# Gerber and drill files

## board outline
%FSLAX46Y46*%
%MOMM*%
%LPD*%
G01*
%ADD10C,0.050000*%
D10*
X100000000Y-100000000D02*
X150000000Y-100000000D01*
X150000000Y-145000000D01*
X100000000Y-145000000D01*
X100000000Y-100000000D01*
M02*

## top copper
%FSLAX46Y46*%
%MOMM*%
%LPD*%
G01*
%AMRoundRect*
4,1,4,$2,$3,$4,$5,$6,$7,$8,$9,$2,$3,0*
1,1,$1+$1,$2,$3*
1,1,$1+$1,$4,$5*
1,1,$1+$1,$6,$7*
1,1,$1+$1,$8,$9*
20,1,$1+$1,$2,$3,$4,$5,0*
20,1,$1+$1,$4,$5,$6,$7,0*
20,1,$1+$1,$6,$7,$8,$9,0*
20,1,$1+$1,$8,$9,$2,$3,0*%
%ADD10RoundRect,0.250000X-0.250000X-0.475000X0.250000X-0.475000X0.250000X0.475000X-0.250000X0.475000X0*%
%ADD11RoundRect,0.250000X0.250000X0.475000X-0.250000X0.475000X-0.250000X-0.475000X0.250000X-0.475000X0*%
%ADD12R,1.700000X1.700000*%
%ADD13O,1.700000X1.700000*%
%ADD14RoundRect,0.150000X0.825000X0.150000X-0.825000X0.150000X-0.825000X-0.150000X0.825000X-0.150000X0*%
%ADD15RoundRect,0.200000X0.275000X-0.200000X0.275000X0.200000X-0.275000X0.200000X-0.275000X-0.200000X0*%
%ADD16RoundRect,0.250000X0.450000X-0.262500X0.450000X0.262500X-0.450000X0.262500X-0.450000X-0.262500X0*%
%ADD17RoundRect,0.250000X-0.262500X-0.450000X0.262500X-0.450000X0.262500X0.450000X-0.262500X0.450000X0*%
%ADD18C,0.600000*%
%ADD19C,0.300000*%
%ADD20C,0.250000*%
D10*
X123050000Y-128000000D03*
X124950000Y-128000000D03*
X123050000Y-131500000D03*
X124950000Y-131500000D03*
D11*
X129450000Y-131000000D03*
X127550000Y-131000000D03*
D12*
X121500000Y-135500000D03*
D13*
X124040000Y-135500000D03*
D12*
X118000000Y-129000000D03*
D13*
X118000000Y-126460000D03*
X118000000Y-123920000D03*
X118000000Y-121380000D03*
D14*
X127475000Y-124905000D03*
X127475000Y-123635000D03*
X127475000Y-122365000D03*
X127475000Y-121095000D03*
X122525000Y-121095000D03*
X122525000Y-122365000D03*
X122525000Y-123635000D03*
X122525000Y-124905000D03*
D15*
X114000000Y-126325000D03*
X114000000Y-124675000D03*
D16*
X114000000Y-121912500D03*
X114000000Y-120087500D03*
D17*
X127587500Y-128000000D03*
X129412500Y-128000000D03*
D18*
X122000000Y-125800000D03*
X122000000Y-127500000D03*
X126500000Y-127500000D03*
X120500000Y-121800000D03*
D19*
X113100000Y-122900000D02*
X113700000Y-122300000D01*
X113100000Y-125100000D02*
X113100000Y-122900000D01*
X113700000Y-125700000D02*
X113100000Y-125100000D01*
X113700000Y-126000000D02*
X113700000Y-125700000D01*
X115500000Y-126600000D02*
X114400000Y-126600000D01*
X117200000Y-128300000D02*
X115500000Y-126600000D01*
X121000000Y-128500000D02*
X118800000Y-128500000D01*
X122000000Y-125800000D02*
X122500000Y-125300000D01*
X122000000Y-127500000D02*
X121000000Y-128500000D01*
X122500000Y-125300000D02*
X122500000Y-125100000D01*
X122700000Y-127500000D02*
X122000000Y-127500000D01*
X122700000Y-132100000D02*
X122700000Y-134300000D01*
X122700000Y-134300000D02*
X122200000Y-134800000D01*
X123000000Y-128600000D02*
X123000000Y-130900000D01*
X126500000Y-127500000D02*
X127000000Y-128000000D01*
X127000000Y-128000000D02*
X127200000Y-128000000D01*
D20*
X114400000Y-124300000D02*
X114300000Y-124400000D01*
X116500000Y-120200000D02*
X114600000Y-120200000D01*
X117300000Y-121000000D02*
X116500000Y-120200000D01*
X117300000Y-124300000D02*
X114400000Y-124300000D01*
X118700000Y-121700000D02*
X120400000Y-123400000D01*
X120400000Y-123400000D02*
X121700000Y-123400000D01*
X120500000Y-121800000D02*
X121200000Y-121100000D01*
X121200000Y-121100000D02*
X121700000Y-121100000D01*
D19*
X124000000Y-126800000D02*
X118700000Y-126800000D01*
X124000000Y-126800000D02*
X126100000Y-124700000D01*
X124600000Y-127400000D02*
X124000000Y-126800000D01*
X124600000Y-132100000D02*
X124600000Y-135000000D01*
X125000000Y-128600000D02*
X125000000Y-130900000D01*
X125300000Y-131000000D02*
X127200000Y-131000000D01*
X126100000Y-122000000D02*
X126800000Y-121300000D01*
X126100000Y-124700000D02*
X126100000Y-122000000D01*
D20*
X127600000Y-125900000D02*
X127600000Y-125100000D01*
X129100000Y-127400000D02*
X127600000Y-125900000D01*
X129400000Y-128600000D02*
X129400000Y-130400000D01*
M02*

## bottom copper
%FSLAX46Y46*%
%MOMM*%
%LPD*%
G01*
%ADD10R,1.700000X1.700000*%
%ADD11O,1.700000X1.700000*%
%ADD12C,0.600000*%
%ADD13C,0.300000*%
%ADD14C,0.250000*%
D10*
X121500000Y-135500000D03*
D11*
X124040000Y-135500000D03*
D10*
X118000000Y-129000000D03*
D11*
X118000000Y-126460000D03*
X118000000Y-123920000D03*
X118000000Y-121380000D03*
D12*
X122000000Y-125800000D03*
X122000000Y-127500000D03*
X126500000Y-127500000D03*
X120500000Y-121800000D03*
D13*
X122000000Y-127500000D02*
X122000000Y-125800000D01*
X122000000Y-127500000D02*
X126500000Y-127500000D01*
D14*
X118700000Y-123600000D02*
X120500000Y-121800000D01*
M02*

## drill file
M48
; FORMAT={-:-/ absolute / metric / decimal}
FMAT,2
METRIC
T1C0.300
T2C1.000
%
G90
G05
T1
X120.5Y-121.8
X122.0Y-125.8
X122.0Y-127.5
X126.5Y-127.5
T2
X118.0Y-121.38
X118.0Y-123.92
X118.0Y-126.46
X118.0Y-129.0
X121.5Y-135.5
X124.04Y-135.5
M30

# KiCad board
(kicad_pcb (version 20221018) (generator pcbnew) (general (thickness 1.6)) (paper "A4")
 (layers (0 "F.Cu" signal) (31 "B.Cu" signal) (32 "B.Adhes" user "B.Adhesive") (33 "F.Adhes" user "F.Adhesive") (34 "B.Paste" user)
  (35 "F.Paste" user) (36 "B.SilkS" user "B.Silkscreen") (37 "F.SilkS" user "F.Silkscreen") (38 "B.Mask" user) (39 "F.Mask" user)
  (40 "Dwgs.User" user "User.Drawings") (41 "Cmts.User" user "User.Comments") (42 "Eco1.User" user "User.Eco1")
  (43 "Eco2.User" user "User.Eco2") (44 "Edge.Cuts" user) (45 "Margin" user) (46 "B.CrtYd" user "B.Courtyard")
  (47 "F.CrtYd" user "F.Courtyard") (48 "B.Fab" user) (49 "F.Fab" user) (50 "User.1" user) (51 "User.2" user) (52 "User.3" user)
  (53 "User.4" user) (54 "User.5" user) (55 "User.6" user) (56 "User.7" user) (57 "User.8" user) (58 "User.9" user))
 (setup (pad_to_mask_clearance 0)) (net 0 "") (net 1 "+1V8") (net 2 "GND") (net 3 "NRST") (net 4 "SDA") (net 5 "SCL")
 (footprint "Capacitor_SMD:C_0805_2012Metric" (layer "F.Cu") (at 124 128)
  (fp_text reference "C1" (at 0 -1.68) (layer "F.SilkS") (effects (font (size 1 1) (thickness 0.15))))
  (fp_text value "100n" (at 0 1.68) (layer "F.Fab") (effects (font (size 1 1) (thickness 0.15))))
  (pad "1" smd roundrect (at -0.95 0) (size 1 1.45) (layers "F.Cu" "F.Paste" "F.Mask") (roundrect_rratio 0.25) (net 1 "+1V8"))
  (pad "2" smd roundrect (at 0.95 0) (size 1 1.45) (layers "F.Cu" "F.Paste" "F.Mask") (roundrect_rratio 0.25) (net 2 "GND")))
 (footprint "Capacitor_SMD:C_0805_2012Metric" (layer "F.Cu") (at 124 131.5)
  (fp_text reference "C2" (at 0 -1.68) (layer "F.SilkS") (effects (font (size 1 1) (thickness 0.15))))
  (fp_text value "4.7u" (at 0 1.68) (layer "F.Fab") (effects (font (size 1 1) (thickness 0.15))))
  (pad "1" smd roundrect (at -0.95 0) (size 1 1.45) (layers "F.Cu" "F.Paste" "F.Mask") (roundrect_rratio 0.25) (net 1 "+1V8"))
  (pad "2" smd roundrect (at 0.95 0) (size 1 1.45) (layers "F.Cu" "F.Paste" "F.Mask") (roundrect_rratio 0.25) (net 2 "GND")))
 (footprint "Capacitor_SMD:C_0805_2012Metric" (layer "F.Cu") (at 128.5 131 180)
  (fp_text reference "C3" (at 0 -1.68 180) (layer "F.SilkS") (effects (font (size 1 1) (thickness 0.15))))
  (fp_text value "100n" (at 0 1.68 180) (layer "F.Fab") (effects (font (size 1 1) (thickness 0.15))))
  (pad "1" smd roundrect (at -0.95 0 180) (size 1 1.45) (layers "F.Cu" "F.Paste" "F.Mask") (roundrect_rratio 0.25) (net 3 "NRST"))
  (pad "2" smd roundrect (at 0.95 0 180) (size 1 1.45) (layers "F.Cu" "F.Paste" "F.Mask") (roundrect_rratio 0.25) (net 2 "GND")))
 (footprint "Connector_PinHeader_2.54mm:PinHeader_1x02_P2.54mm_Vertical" (layer "F.Cu") (at 121.5 135.5 90)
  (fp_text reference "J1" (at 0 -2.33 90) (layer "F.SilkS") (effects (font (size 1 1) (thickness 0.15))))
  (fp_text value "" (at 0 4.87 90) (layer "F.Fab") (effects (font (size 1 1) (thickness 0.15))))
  (pad "1" thru_hole rect (at 0 0 90) (size 1.7 1.7) (drill 1) (layers "*.Cu" "*.Mask") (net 1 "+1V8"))
  (pad "2" thru_hole oval (at 0 2.54 90) (size 1.7 1.7) (drill 1) (layers "*.Cu" "*.Mask") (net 2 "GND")))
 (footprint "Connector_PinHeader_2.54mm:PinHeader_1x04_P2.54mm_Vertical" (layer "F.Cu") (at 118 129 180)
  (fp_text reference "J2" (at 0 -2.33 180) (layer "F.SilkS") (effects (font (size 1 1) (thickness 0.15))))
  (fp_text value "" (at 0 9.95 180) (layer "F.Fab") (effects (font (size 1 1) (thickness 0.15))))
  (pad "1" thru_hole rect (at 0 0 180) (size 1.7 1.7) (drill 1) (layers "*.Cu" "*.Mask") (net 1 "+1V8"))
  (pad "2" thru_hole oval (at 0 2.54 180) (size 1.7 1.7) (drill 1) (layers "*.Cu" "*.Mask") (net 2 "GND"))
  (pad "3" thru_hole oval (at 0 5.08 180) (size 1.7 1.7) (drill 1) (layers "*.Cu" "*.Mask") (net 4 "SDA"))
  (pad "4" thru_hole oval (at 0 7.62 180) (size 1.7 1.7) (drill 1) (layers "*.Cu" "*.Mask") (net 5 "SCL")))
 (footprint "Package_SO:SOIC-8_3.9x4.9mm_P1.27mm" (layer "F.Cu") (at 125 123 180)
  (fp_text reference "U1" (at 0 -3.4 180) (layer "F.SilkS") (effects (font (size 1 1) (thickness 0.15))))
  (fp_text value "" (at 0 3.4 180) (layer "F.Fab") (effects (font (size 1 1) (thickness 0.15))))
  (pad "1" smd roundrect (at -2.475 -1.905 180) (size 1.95 0.6) (layers "F.Cu" "F.Paste" "F.Mask") (roundrect_rratio 0.25) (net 3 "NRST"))
  (pad "2" smd roundrect (at -2.475 -0.635 180) (size 1.95 0.6) (layers "F.Cu" "F.Paste" "F.Mask") (roundrect_rratio 0.25))
  (pad "3" smd roundrect (at -2.475 0.635 180) (size 1.95 0.6) (layers "F.Cu" "F.Paste" "F.Mask") (roundrect_rratio 0.25))
  (pad "4" smd roundrect (at -2.475 1.905 180) (size 1.95 0.6) (layers "F.Cu" "F.Paste" "F.Mask") (roundrect_rratio 0.25) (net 2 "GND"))
  (pad "5" smd roundrect (at 2.475 1.905 180) (size 1.95 0.6) (layers "F.Cu" "F.Paste" "F.Mask") (roundrect_rratio 0.25) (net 4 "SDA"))
  (pad "6" smd roundrect (at 2.475 0.635 180) (size 1.95 0.6) (layers "F.Cu" "F.Paste" "F.Mask") (roundrect_rratio 0.25))
  (pad "7" smd roundrect (at 2.475 -0.635 180) (size 1.95 0.6) (layers "F.Cu" "F.Paste" "F.Mask") (roundrect_rratio 0.25) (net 5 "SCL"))
  (pad "8" smd roundrect (at 2.475 -1.905 180) (size 1.95 0.6) (layers "F.Cu" "F.Paste" "F.Mask") (roundrect_rratio 0.25) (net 1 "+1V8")))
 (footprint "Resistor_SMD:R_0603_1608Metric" (layer "F.Cu") (at 114 125.5 90)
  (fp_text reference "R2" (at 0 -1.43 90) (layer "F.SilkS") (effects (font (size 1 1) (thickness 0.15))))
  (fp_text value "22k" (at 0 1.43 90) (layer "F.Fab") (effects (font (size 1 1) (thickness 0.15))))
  (pad "1" smd roundrect (at -0.825 0 90) (size 0.8 0.95) (layers "F.Cu" "F.Paste" "F.Mask") (roundrect_rratio 0.25) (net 1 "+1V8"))
  (pad "2" smd roundrect (at 0.825 0 90) (size 0.8 0.95) (layers "F.Cu" "F.Paste" "F.Mask") (roundrect_rratio 0.25) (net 4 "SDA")))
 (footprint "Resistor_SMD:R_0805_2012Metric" (layer "F.Cu") (at 114 121 90)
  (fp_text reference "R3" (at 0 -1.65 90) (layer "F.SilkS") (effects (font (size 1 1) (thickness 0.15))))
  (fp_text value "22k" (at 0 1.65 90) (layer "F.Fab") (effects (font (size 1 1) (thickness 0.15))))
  (pad "1" smd roundrect (at -0.9125 0 90) (size 1.025 1.4) (layers "F.Cu" "F.Paste" "F.Mask") (roundrect_rratio 0.243902) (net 1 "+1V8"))
  (pad "2" smd roundrect (at 0.9125 0 90) (size 1.025 1.4) (layers "F.Cu" "F.Paste" "F.Mask") (roundrect_rratio 0.243902) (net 5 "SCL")))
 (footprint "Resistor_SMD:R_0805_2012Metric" (layer "F.Cu") (at 128.5 128)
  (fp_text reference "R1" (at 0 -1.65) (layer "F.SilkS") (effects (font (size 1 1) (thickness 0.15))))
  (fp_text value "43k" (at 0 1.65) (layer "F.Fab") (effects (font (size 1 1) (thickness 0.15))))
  (pad "1" smd roundrect (at -0.9125 0) (size 1.025 1.4) (layers "F.Cu" "F.Paste" "F.Mask") (roundrect_rratio 0.243902) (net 1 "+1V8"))
  (pad "2" smd roundrect (at 0.9125 0) (size 1.025 1.4) (layers "F.Cu" "F.Paste" "F.Mask") (roundrect_rratio 0.243902) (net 3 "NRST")))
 (gr_rect (start 100 100) (end 150 145) (stroke (width 0.05) (type default)) (fill none) (layer "Edge.Cuts"))
 (segment (start 113.1 122.9) (end 113.7 122.3) (width 0.3) (layer "F.Cu") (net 1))
 (segment (start 113.1 125.1) (end 113.1 122.9) (width 0.3) (layer "F.Cu") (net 1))
 (segment (start 113.7 125.7) (end 113.1 125.1) (width 0.3) (layer "F.Cu") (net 1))
 (segment (start 113.7 126) (end 113.7 125.7) (width 0.3) (layer "F.Cu") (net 1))
 (segment (start 115.5 126.6) (end 114.4 126.6) (width 0.3) (layer "F.Cu") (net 1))
 (segment (start 117.2 128.3) (end 115.5 126.6) (width 0.3) (layer "F.Cu") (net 1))
 (segment (start 121 128.5) (end 118.8 128.5) (width 0.3) (layer "F.Cu") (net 1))
 (segment (start 122 125.8) (end 122.5 125.3) (width 0.3) (layer "F.Cu") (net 1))
 (segment (start 122 127.5) (end 121 128.5) (width 0.3) (layer "F.Cu") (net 1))
 (segment (start 122.5 125.3) (end 122.5 125.1) (width 0.3) (layer "F.Cu") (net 1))
 (segment (start 122.7 127.5) (end 122 127.5) (width 0.3) (layer "F.Cu") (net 1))
 (segment (start 122.7 132.1) (end 122.7 134.3) (width 0.3) (layer "F.Cu") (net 1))
 (segment (start 122.7 134.3) (end 122.2 134.8) (width 0.3) (layer "F.Cu") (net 1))
 (segment (start 123 128.6) (end 123 130.9) (width 0.3) (layer "F.Cu") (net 1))
 (segment (start 126.5 127.5) (end 127 128) (width 0.3) (layer "F.Cu") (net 1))
 (segment (start 127 128) (end 127.2 128) (width 0.3) (layer "F.Cu") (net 1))
 (via (at 122 125.8) (size 0.6) (drill 0.3) (layers "F.Cu" "B.Cu") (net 1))
 (via (at 122 127.5) (size 0.6) (drill 0.3) (layers "F.Cu" "B.Cu") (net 1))
 (via (at 126.5 127.5) (size 0.6) (drill 0.3) (layers "F.Cu" "B.Cu") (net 1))
 (segment (start 114.4 124.3) (end 114.3 124.4) (width 0.25) (layer "F.Cu") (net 4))
 (segment (start 116.5 120.2) (end 114.6 120.2) (width 0.25) (layer "F.Cu") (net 5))
 (segment (start 117.3 121) (end 116.5 120.2) (width 0.25) (layer "F.Cu") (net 5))
 (segment (start 117.3 124.3) (end 114.4 124.3) (width 0.25) (layer "F.Cu") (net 4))
 (segment (start 118.7 121.7) (end 120.4 123.4) (width 0.25) (layer "F.Cu") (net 5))
 (segment (start 120.4 123.4) (end 121.7 123.4) (width 0.25) (layer "F.Cu") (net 5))
 (segment (start 120.5 121.8) (end 121.2 121.1) (width 0.25) (layer "F.Cu") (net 4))
 (segment (start 121.2 121.1) (end 121.7 121.1) (width 0.25) (layer "F.Cu") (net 4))
 (segment (start 122 127.5) (end 122 125.8) (width 0.3) (layer "B.Cu") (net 1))
 (segment (start 122 127.5) (end 126.5 127.5) (width 0.3) (layer "B.Cu") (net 1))
 (segment (start 124 126.8) (end 118.7 126.8) (width 0.3) (layer "F.Cu") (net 2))
 (segment (start 124 126.8) (end 126.1 124.7) (width 0.3) (layer "F.Cu") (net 2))
 (segment (start 124.6 127.4) (end 124 126.8) (width 0.3) (layer "F.Cu") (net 2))
 (segment (start 124.6 132.1) (end 124.6 135) (width 0.3) (layer "F.Cu") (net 2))
 (segment (start 125 128.6) (end 125 130.9) (width 0.3) (layer "F.Cu") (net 2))
 (segment (start 125.3 131) (end 127.2 131) (width 0.3) (layer "F.Cu") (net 2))
 (segment (start 126.1 122) (end 126.8 121.3) (width 0.3) (layer "F.Cu") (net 2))
 (segment (start 126.1 124.7) (end 126.1 122) (width 0.3) (layer "F.Cu") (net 2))
 (segment (start 127.6 125.9) (end 127.6 125.1) (width 0.25) (layer "F.Cu") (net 3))
 (segment (start 129.1 127.4) (end 127.6 125.9) (width 0.25) (layer "F.Cu") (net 3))
 (segment (start 129.4 128.6) (end 129.4 130.4) (width 0.25) (layer "F.Cu") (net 3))
 (via (at 120.5 121.8) (size 0.6) (drill 0.3) (layers "F.Cu" "B.Cu") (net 4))
 (segment (start 118.7 123.6) (end 120.5 121.8) (width 0.25) (layer "B.Cu") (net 4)))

